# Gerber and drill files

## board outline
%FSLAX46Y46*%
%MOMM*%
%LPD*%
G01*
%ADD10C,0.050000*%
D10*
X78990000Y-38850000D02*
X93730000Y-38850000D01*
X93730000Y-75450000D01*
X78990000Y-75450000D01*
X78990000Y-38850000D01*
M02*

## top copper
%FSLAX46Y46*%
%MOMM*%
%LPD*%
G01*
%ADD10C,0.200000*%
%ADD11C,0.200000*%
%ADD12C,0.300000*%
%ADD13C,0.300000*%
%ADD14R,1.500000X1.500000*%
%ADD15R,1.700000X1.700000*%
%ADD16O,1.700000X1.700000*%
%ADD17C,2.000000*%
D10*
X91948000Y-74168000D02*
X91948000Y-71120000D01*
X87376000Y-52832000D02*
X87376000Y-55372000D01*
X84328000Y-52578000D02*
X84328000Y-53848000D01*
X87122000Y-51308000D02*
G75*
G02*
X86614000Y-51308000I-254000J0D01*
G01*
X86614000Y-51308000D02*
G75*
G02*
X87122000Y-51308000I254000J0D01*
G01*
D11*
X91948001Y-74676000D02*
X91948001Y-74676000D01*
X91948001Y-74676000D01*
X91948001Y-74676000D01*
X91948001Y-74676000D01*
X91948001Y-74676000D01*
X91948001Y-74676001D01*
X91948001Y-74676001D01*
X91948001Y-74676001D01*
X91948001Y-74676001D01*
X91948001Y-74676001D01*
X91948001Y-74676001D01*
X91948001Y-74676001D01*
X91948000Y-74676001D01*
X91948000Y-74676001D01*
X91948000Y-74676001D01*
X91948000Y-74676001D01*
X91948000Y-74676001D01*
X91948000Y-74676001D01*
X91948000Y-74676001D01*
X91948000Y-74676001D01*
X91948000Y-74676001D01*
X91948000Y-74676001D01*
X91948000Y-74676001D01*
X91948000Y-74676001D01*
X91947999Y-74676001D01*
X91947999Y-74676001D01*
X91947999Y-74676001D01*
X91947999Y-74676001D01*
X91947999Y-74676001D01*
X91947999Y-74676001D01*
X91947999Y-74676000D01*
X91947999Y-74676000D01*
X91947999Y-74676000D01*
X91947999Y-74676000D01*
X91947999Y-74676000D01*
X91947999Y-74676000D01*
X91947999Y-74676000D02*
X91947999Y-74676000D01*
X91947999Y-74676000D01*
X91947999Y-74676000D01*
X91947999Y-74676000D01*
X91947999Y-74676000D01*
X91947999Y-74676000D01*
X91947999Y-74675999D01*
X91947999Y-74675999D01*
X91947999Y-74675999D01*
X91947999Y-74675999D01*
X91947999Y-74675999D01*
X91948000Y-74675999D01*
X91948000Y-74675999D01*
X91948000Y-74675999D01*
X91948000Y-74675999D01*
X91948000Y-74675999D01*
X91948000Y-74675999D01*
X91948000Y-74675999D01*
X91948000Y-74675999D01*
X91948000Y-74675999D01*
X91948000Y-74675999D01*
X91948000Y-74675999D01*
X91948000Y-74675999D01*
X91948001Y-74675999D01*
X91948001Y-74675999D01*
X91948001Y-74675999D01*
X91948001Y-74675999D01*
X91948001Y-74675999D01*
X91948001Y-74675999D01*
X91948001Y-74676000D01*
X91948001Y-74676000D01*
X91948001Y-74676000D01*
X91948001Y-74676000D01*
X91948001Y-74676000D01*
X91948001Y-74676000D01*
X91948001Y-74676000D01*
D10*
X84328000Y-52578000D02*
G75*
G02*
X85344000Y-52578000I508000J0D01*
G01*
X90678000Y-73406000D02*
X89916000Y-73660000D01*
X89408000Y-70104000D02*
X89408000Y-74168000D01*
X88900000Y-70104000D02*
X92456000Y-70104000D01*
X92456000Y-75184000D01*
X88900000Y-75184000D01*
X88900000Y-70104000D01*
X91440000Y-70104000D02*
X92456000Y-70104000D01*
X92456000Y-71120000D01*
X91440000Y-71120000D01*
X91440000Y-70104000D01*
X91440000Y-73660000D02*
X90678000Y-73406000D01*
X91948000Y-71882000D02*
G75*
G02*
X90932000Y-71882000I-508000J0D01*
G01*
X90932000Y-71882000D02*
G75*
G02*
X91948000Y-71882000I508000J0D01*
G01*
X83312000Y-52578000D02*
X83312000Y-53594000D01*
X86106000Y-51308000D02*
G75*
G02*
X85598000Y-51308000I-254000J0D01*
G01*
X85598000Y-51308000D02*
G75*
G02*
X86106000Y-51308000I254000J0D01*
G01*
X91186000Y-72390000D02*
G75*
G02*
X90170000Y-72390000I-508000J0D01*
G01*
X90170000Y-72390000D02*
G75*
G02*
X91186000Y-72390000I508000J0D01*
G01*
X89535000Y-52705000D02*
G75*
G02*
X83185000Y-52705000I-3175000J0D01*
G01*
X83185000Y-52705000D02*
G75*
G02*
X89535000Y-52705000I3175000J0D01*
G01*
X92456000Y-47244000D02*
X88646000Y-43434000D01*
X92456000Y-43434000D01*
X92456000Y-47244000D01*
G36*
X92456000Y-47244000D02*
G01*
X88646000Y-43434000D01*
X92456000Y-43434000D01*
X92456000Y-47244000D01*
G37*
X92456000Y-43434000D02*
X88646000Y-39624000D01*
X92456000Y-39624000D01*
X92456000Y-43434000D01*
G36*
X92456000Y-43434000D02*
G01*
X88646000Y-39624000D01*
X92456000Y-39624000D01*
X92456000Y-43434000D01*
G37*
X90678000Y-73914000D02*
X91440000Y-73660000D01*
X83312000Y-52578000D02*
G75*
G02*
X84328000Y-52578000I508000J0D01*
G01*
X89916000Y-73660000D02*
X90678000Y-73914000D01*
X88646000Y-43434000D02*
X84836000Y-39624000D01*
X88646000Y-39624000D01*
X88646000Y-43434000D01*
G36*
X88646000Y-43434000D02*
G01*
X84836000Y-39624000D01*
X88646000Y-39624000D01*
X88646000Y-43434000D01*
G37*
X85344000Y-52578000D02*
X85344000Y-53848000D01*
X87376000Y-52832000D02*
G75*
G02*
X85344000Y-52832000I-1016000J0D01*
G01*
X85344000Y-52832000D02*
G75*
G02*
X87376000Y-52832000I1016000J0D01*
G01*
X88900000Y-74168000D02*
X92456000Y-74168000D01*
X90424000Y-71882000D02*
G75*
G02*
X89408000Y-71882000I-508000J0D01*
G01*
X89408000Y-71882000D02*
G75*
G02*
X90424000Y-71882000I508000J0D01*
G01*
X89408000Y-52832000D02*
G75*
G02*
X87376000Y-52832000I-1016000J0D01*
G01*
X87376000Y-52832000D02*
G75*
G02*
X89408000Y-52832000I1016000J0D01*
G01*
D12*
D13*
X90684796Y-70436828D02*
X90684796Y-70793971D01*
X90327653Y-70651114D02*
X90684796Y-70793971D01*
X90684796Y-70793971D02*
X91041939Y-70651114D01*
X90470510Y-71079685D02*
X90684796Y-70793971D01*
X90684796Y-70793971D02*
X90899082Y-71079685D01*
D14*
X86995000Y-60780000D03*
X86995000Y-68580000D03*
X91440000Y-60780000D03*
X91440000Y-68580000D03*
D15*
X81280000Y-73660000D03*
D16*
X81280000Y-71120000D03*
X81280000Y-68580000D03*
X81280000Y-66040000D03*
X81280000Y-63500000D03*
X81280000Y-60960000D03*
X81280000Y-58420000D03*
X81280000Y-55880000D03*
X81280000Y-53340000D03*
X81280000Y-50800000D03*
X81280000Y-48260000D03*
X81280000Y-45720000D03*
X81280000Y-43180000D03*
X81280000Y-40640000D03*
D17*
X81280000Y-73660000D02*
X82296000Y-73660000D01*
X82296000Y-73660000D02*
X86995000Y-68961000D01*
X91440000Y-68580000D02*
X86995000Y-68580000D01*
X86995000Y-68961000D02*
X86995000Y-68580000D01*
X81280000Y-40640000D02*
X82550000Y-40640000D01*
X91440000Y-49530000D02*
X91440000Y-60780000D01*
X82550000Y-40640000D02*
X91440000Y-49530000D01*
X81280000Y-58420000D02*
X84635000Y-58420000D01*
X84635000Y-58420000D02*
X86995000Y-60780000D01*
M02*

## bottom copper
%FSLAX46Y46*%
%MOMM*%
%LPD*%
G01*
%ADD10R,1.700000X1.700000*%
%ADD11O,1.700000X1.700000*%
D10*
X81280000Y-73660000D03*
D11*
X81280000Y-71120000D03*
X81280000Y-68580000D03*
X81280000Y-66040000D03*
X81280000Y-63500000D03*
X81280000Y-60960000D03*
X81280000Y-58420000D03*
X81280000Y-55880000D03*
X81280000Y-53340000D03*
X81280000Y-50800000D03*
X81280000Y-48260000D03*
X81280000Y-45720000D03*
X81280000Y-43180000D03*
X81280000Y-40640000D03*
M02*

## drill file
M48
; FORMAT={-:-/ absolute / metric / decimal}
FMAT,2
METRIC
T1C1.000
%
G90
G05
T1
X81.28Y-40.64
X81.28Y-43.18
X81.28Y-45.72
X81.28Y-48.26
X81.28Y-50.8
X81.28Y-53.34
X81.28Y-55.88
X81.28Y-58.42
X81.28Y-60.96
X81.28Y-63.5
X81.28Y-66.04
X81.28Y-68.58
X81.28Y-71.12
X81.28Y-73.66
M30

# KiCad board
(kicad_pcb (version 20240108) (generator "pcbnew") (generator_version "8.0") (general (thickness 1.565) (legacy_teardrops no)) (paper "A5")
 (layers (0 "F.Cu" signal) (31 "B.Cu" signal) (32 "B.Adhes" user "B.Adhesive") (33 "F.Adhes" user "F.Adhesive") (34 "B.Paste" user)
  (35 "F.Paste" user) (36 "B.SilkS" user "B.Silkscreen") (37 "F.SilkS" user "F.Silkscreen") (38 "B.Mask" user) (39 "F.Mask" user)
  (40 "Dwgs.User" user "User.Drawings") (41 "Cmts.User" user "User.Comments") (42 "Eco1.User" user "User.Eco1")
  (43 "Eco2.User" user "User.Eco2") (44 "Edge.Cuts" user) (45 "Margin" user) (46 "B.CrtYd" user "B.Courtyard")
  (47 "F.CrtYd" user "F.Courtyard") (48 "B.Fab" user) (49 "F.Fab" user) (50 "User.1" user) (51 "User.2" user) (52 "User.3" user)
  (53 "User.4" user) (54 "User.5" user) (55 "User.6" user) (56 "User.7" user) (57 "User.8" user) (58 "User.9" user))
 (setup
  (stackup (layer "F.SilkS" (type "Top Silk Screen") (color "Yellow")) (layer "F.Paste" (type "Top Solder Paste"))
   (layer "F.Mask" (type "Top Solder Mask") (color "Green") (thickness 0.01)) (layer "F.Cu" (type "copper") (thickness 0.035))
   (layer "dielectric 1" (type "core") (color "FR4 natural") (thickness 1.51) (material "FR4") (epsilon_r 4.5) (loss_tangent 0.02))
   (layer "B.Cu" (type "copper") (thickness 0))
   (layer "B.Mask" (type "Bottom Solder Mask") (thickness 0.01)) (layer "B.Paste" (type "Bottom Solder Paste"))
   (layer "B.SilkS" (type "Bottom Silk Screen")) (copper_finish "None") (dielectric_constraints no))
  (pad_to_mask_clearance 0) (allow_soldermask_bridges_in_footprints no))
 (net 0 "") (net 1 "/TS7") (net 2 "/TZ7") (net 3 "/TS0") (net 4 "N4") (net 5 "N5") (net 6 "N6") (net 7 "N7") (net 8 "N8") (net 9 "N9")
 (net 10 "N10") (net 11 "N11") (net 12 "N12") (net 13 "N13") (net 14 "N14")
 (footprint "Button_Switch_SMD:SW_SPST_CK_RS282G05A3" (layer "F.Cu") (at 86.995 64.68 -90)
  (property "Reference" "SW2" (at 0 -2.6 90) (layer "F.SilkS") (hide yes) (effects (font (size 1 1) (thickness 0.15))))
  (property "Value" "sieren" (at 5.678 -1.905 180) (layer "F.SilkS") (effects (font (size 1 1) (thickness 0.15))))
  (pad "1" smd rect (at -3.9 0 270) (size 1.5 1.5) (layers "F.Cu" "F.Paste" "F.Mask") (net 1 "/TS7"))
  (pad "2" smd rect (at 3.9 0 270) (size 1.5 1.5) (layers "F.Cu" "F.Paste" "F.Mask") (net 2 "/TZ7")))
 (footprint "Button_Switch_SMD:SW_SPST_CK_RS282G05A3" (layer "F.Cu") (at 91.44 64.68 -90)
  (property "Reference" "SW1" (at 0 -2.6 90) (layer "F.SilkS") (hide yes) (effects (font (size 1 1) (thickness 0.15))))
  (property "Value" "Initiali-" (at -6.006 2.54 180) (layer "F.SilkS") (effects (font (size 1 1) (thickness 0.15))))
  (pad "1" smd rect (at -3.9 0 270) (size 1.5 1.5) (layers "F.Cu" "F.Paste" "F.Mask") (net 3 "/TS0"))
  (pad "2" smd rect (at 3.9 0 270) (size 1.5 1.5) (layers "F.Cu" "F.Paste" "F.Mask") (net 2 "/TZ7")))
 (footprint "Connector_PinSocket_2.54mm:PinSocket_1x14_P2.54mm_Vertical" (layer "B.Cu") (at 81.28 73.66)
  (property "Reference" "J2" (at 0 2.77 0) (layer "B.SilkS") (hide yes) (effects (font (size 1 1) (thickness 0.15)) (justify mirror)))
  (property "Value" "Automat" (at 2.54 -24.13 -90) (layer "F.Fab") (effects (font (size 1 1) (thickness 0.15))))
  (pad "1" thru_hole rect (at 0 0) (size 1.7 1.7) (drill 1) (layers "*.Cu" "*.Mask") (remove_unused_layers no) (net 2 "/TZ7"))
  (pad "2" thru_hole oval (at 0 -2.54) (size 1.7 1.7) (drill 1) (layers "*.Cu" "*.Mask") (remove_unused_layers no) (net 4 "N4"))
  (pad "3" thru_hole oval (at 0 -5.08) (size 1.7 1.7) (drill 1) (layers "*.Cu" "*.Mask") (remove_unused_layers no) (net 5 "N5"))
  (pad "4" thru_hole oval (at 0 -7.62) (size 1.7 1.7) (drill 1) (layers "*.Cu" "*.Mask") (remove_unused_layers no) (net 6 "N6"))
  (pad "5" thru_hole oval (at 0 -10.16) (size 1.7 1.7) (drill 1) (layers "*.Cu" "*.Mask") (remove_unused_layers no) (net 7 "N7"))
  (pad "6" thru_hole oval (at 0 -12.7) (size 1.7 1.7) (drill 1) (layers "*.Cu" "*.Mask") (remove_unused_layers no) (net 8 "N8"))
  (pad "7" thru_hole oval (at 0 -15.24) (size 1.7 1.7) (drill 1) (layers "*.Cu" "*.Mask") (remove_unused_layers no) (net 1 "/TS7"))
  (pad "8" thru_hole oval (at 0 -17.78) (size 1.7 1.7) (drill 1) (layers "*.Cu" "*.Mask") (remove_unused_layers no) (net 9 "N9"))
  (pad "9" thru_hole oval (at 0 -20.32) (size 1.7 1.7) (drill 1) (layers "*.Cu" "*.Mask") (remove_unused_layers no) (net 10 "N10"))
  (pad "10" thru_hole oval (at 0 -22.86) (size 1.7 1.7) (drill 1) (layers "*.Cu" "*.Mask") (remove_unused_layers no) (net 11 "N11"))
  (pad "11" thru_hole oval (at 0 -25.4) (size 1.7 1.7) (drill 1) (layers "*.Cu" "*.Mask") (remove_unused_layers no) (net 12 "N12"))
  (pad "12" thru_hole oval (at 0 -27.94) (size 1.7 1.7) (drill 1) (layers "*.Cu" "*.Mask") (remove_unused_layers no) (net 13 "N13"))
  (pad "13" thru_hole oval (at 0 -30.48) (size 1.7 1.7) (drill 1) (layers "*.Cu" "*.Mask") (remove_unused_layers no) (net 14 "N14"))
  (pad "14" thru_hole oval (at 0 -33.02) (size 1.7 1.7) (drill 1) (layers "*.Cu" "*.Mask") (remove_unused_layers no) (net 3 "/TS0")))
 (gr_line (start 91.948 74.168) (end 91.948 71.12) (stroke (width 0.2) (type default)) (layer "F.Cu"))
 (gr_line (start 87.376 52.832) (end 87.376 55.372) (stroke (width 0.2) (type default)) (layer "F.Cu"))
 (gr_line (start 84.328 52.578) (end 84.328 53.848) (stroke (width 0.2) (type default)) (layer "F.Cu"))
 (gr_circle (center 86.868 51.308) (end 87.122 51.308) (stroke (width 0.2) (type default)) (fill none) (layer "F.Cu"))
 (gr_circle (center 91.948 74.676) (end 91.948 74.676) (stroke (width 0.2) (type default)) (fill none) (layer "F.Cu"))
 (gr_arc (start 84.328 52.578) (mid 84.836 52.07) (end 85.344 52.578) (stroke (width 0.2) (type default)) (layer "F.Cu"))
 (gr_line (start 90.678 73.406) (end 89.916 73.66) (stroke (width 0.2) (type default)) (layer "F.Cu"))
 (gr_line (start 89.408 70.104) (end 89.408 74.168) (stroke (width 0.2) (type default)) (layer "F.Cu"))
 (gr_rect (start 88.9 70.104) (end 92.456 75.184) (stroke (width 0.2) (type default)) (fill none) (layer "F.Cu"))
 (gr_rect (start 91.44 70.104) (end 92.456 71.12) (stroke (width 0.2) (type default)) (fill none) (layer "F.Cu"))
 (gr_line (start 91.44 73.66) (end 90.678 73.406) (stroke (width 0.2) (type default)) (layer "F.Cu"))
 (gr_circle (center 91.44 71.882) (end 90.932 71.882) (stroke (width 0.2) (type default)) (fill none) (layer "F.Cu"))
 (gr_line (start 83.312 52.578) (end 83.312 53.594) (stroke (width 0.2) (type default)) (layer "F.Cu"))
 (gr_circle (center 85.852 51.308) (end 86.106 51.308) (stroke (width 0.2) (type default)) (fill none) (layer "F.Cu"))
 (gr_circle (center 90.678 72.39) (end 90.678 71.882) (stroke (width 0.2) (type default)) (fill none) (layer "F.Cu"))
 (gr_circle (center 86.36 52.705) (end 86.36 49.53) (stroke (width 0.2) (type default)) (fill none) (layer "F.Cu"))
 (gr_poly (pts (xy 92.456 47.244) (xy 88.646 43.434) (xy 92.456 43.434)) (stroke (width 0.2) (type solid)) (fill solid) (layer "F.Cu"))
 (gr_poly (pts (xy 92.456 43.434) (xy 88.646 39.624) (xy 92.456 39.624)) (stroke (width 0.2) (type solid)) (fill solid) (layer "F.Cu"))
 (gr_line (start 90.678 73.914) (end 91.44 73.66) (stroke (width 0.2) (type default)) (layer "F.Cu"))
 (gr_arc (start 83.312 52.578) (mid 83.82 52.07) (end 84.328 52.578) (stroke (width 0.2) (type default)) (layer "F.Cu"))
 (gr_line (start 89.916 73.66) (end 90.678 73.914) (stroke (width 0.2) (type default)) (layer "F.Cu"))
 (gr_poly (pts (xy 88.646 43.434) (xy 84.836 39.624) (xy 88.646 39.624)) (stroke (width 0.2) (type solid)) (fill solid) (layer "F.Cu"))
 (gr_line (start 85.344 52.578) (end 85.344 53.848) (stroke (width 0.2) (type default)) (layer "F.Cu"))
 (gr_circle (center 86.36 52.832) (end 85.344 52.832) (stroke (width 0.2) (type default)) (fill none) (layer "F.Cu"))
 (gr_line (start 88.9 74.168) (end 92.456 74.168) (stroke (width 0.2) (type default)) (layer "F.Cu"))
 (gr_circle (center 89.916 71.882) (end 89.408 71.882) (stroke (width 0.2) (type default)) (fill none) (layer "F.Cu"))
 (gr_circle (center 88.392 52.832) (end 87.376 52.832) (stroke (width 0.2) (type default)) (fill none) (layer "F.Cu"))
 (gr_rect (start 78.99 38.85) (end 93.73 75.45) (stroke (width 0.05) (type default)) (fill none) (layer "Edge.Cuts"))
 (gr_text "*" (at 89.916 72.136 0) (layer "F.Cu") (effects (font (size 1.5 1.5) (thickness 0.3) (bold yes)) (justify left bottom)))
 (segment (start 81.28 73.66) (end 82.296 73.66) (width 2) (layer "F.Cu") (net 2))
 (segment (start 82.296 73.66) (end 86.995 68.961) (width 2) (layer "F.Cu") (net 2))
 (segment (start 91.44 68.58) (end 86.995 68.58) (width 2) (layer "F.Cu") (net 2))
 (segment (start 86.995 68.961) (end 86.995 68.58) (width 2) (layer "F.Cu") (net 2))
 (segment (start 81.28 40.64) (end 82.55 40.64) (width 2) (layer "F.Cu") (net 3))
 (segment (start 91.44 49.53) (end 91.44 60.78) (width 2) (layer "F.Cu") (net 3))
 (segment (start 82.55 40.64) (end 91.44 49.53) (width 2) (layer "F.Cu") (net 3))
 (segment (start 81.28 58.42) (end 84.635 58.42) (width 2) (layer "F.Cu") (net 1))
 (segment (start 84.635 58.42) (end 86.995 60.78) (width 2) (layer "F.Cu") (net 1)))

